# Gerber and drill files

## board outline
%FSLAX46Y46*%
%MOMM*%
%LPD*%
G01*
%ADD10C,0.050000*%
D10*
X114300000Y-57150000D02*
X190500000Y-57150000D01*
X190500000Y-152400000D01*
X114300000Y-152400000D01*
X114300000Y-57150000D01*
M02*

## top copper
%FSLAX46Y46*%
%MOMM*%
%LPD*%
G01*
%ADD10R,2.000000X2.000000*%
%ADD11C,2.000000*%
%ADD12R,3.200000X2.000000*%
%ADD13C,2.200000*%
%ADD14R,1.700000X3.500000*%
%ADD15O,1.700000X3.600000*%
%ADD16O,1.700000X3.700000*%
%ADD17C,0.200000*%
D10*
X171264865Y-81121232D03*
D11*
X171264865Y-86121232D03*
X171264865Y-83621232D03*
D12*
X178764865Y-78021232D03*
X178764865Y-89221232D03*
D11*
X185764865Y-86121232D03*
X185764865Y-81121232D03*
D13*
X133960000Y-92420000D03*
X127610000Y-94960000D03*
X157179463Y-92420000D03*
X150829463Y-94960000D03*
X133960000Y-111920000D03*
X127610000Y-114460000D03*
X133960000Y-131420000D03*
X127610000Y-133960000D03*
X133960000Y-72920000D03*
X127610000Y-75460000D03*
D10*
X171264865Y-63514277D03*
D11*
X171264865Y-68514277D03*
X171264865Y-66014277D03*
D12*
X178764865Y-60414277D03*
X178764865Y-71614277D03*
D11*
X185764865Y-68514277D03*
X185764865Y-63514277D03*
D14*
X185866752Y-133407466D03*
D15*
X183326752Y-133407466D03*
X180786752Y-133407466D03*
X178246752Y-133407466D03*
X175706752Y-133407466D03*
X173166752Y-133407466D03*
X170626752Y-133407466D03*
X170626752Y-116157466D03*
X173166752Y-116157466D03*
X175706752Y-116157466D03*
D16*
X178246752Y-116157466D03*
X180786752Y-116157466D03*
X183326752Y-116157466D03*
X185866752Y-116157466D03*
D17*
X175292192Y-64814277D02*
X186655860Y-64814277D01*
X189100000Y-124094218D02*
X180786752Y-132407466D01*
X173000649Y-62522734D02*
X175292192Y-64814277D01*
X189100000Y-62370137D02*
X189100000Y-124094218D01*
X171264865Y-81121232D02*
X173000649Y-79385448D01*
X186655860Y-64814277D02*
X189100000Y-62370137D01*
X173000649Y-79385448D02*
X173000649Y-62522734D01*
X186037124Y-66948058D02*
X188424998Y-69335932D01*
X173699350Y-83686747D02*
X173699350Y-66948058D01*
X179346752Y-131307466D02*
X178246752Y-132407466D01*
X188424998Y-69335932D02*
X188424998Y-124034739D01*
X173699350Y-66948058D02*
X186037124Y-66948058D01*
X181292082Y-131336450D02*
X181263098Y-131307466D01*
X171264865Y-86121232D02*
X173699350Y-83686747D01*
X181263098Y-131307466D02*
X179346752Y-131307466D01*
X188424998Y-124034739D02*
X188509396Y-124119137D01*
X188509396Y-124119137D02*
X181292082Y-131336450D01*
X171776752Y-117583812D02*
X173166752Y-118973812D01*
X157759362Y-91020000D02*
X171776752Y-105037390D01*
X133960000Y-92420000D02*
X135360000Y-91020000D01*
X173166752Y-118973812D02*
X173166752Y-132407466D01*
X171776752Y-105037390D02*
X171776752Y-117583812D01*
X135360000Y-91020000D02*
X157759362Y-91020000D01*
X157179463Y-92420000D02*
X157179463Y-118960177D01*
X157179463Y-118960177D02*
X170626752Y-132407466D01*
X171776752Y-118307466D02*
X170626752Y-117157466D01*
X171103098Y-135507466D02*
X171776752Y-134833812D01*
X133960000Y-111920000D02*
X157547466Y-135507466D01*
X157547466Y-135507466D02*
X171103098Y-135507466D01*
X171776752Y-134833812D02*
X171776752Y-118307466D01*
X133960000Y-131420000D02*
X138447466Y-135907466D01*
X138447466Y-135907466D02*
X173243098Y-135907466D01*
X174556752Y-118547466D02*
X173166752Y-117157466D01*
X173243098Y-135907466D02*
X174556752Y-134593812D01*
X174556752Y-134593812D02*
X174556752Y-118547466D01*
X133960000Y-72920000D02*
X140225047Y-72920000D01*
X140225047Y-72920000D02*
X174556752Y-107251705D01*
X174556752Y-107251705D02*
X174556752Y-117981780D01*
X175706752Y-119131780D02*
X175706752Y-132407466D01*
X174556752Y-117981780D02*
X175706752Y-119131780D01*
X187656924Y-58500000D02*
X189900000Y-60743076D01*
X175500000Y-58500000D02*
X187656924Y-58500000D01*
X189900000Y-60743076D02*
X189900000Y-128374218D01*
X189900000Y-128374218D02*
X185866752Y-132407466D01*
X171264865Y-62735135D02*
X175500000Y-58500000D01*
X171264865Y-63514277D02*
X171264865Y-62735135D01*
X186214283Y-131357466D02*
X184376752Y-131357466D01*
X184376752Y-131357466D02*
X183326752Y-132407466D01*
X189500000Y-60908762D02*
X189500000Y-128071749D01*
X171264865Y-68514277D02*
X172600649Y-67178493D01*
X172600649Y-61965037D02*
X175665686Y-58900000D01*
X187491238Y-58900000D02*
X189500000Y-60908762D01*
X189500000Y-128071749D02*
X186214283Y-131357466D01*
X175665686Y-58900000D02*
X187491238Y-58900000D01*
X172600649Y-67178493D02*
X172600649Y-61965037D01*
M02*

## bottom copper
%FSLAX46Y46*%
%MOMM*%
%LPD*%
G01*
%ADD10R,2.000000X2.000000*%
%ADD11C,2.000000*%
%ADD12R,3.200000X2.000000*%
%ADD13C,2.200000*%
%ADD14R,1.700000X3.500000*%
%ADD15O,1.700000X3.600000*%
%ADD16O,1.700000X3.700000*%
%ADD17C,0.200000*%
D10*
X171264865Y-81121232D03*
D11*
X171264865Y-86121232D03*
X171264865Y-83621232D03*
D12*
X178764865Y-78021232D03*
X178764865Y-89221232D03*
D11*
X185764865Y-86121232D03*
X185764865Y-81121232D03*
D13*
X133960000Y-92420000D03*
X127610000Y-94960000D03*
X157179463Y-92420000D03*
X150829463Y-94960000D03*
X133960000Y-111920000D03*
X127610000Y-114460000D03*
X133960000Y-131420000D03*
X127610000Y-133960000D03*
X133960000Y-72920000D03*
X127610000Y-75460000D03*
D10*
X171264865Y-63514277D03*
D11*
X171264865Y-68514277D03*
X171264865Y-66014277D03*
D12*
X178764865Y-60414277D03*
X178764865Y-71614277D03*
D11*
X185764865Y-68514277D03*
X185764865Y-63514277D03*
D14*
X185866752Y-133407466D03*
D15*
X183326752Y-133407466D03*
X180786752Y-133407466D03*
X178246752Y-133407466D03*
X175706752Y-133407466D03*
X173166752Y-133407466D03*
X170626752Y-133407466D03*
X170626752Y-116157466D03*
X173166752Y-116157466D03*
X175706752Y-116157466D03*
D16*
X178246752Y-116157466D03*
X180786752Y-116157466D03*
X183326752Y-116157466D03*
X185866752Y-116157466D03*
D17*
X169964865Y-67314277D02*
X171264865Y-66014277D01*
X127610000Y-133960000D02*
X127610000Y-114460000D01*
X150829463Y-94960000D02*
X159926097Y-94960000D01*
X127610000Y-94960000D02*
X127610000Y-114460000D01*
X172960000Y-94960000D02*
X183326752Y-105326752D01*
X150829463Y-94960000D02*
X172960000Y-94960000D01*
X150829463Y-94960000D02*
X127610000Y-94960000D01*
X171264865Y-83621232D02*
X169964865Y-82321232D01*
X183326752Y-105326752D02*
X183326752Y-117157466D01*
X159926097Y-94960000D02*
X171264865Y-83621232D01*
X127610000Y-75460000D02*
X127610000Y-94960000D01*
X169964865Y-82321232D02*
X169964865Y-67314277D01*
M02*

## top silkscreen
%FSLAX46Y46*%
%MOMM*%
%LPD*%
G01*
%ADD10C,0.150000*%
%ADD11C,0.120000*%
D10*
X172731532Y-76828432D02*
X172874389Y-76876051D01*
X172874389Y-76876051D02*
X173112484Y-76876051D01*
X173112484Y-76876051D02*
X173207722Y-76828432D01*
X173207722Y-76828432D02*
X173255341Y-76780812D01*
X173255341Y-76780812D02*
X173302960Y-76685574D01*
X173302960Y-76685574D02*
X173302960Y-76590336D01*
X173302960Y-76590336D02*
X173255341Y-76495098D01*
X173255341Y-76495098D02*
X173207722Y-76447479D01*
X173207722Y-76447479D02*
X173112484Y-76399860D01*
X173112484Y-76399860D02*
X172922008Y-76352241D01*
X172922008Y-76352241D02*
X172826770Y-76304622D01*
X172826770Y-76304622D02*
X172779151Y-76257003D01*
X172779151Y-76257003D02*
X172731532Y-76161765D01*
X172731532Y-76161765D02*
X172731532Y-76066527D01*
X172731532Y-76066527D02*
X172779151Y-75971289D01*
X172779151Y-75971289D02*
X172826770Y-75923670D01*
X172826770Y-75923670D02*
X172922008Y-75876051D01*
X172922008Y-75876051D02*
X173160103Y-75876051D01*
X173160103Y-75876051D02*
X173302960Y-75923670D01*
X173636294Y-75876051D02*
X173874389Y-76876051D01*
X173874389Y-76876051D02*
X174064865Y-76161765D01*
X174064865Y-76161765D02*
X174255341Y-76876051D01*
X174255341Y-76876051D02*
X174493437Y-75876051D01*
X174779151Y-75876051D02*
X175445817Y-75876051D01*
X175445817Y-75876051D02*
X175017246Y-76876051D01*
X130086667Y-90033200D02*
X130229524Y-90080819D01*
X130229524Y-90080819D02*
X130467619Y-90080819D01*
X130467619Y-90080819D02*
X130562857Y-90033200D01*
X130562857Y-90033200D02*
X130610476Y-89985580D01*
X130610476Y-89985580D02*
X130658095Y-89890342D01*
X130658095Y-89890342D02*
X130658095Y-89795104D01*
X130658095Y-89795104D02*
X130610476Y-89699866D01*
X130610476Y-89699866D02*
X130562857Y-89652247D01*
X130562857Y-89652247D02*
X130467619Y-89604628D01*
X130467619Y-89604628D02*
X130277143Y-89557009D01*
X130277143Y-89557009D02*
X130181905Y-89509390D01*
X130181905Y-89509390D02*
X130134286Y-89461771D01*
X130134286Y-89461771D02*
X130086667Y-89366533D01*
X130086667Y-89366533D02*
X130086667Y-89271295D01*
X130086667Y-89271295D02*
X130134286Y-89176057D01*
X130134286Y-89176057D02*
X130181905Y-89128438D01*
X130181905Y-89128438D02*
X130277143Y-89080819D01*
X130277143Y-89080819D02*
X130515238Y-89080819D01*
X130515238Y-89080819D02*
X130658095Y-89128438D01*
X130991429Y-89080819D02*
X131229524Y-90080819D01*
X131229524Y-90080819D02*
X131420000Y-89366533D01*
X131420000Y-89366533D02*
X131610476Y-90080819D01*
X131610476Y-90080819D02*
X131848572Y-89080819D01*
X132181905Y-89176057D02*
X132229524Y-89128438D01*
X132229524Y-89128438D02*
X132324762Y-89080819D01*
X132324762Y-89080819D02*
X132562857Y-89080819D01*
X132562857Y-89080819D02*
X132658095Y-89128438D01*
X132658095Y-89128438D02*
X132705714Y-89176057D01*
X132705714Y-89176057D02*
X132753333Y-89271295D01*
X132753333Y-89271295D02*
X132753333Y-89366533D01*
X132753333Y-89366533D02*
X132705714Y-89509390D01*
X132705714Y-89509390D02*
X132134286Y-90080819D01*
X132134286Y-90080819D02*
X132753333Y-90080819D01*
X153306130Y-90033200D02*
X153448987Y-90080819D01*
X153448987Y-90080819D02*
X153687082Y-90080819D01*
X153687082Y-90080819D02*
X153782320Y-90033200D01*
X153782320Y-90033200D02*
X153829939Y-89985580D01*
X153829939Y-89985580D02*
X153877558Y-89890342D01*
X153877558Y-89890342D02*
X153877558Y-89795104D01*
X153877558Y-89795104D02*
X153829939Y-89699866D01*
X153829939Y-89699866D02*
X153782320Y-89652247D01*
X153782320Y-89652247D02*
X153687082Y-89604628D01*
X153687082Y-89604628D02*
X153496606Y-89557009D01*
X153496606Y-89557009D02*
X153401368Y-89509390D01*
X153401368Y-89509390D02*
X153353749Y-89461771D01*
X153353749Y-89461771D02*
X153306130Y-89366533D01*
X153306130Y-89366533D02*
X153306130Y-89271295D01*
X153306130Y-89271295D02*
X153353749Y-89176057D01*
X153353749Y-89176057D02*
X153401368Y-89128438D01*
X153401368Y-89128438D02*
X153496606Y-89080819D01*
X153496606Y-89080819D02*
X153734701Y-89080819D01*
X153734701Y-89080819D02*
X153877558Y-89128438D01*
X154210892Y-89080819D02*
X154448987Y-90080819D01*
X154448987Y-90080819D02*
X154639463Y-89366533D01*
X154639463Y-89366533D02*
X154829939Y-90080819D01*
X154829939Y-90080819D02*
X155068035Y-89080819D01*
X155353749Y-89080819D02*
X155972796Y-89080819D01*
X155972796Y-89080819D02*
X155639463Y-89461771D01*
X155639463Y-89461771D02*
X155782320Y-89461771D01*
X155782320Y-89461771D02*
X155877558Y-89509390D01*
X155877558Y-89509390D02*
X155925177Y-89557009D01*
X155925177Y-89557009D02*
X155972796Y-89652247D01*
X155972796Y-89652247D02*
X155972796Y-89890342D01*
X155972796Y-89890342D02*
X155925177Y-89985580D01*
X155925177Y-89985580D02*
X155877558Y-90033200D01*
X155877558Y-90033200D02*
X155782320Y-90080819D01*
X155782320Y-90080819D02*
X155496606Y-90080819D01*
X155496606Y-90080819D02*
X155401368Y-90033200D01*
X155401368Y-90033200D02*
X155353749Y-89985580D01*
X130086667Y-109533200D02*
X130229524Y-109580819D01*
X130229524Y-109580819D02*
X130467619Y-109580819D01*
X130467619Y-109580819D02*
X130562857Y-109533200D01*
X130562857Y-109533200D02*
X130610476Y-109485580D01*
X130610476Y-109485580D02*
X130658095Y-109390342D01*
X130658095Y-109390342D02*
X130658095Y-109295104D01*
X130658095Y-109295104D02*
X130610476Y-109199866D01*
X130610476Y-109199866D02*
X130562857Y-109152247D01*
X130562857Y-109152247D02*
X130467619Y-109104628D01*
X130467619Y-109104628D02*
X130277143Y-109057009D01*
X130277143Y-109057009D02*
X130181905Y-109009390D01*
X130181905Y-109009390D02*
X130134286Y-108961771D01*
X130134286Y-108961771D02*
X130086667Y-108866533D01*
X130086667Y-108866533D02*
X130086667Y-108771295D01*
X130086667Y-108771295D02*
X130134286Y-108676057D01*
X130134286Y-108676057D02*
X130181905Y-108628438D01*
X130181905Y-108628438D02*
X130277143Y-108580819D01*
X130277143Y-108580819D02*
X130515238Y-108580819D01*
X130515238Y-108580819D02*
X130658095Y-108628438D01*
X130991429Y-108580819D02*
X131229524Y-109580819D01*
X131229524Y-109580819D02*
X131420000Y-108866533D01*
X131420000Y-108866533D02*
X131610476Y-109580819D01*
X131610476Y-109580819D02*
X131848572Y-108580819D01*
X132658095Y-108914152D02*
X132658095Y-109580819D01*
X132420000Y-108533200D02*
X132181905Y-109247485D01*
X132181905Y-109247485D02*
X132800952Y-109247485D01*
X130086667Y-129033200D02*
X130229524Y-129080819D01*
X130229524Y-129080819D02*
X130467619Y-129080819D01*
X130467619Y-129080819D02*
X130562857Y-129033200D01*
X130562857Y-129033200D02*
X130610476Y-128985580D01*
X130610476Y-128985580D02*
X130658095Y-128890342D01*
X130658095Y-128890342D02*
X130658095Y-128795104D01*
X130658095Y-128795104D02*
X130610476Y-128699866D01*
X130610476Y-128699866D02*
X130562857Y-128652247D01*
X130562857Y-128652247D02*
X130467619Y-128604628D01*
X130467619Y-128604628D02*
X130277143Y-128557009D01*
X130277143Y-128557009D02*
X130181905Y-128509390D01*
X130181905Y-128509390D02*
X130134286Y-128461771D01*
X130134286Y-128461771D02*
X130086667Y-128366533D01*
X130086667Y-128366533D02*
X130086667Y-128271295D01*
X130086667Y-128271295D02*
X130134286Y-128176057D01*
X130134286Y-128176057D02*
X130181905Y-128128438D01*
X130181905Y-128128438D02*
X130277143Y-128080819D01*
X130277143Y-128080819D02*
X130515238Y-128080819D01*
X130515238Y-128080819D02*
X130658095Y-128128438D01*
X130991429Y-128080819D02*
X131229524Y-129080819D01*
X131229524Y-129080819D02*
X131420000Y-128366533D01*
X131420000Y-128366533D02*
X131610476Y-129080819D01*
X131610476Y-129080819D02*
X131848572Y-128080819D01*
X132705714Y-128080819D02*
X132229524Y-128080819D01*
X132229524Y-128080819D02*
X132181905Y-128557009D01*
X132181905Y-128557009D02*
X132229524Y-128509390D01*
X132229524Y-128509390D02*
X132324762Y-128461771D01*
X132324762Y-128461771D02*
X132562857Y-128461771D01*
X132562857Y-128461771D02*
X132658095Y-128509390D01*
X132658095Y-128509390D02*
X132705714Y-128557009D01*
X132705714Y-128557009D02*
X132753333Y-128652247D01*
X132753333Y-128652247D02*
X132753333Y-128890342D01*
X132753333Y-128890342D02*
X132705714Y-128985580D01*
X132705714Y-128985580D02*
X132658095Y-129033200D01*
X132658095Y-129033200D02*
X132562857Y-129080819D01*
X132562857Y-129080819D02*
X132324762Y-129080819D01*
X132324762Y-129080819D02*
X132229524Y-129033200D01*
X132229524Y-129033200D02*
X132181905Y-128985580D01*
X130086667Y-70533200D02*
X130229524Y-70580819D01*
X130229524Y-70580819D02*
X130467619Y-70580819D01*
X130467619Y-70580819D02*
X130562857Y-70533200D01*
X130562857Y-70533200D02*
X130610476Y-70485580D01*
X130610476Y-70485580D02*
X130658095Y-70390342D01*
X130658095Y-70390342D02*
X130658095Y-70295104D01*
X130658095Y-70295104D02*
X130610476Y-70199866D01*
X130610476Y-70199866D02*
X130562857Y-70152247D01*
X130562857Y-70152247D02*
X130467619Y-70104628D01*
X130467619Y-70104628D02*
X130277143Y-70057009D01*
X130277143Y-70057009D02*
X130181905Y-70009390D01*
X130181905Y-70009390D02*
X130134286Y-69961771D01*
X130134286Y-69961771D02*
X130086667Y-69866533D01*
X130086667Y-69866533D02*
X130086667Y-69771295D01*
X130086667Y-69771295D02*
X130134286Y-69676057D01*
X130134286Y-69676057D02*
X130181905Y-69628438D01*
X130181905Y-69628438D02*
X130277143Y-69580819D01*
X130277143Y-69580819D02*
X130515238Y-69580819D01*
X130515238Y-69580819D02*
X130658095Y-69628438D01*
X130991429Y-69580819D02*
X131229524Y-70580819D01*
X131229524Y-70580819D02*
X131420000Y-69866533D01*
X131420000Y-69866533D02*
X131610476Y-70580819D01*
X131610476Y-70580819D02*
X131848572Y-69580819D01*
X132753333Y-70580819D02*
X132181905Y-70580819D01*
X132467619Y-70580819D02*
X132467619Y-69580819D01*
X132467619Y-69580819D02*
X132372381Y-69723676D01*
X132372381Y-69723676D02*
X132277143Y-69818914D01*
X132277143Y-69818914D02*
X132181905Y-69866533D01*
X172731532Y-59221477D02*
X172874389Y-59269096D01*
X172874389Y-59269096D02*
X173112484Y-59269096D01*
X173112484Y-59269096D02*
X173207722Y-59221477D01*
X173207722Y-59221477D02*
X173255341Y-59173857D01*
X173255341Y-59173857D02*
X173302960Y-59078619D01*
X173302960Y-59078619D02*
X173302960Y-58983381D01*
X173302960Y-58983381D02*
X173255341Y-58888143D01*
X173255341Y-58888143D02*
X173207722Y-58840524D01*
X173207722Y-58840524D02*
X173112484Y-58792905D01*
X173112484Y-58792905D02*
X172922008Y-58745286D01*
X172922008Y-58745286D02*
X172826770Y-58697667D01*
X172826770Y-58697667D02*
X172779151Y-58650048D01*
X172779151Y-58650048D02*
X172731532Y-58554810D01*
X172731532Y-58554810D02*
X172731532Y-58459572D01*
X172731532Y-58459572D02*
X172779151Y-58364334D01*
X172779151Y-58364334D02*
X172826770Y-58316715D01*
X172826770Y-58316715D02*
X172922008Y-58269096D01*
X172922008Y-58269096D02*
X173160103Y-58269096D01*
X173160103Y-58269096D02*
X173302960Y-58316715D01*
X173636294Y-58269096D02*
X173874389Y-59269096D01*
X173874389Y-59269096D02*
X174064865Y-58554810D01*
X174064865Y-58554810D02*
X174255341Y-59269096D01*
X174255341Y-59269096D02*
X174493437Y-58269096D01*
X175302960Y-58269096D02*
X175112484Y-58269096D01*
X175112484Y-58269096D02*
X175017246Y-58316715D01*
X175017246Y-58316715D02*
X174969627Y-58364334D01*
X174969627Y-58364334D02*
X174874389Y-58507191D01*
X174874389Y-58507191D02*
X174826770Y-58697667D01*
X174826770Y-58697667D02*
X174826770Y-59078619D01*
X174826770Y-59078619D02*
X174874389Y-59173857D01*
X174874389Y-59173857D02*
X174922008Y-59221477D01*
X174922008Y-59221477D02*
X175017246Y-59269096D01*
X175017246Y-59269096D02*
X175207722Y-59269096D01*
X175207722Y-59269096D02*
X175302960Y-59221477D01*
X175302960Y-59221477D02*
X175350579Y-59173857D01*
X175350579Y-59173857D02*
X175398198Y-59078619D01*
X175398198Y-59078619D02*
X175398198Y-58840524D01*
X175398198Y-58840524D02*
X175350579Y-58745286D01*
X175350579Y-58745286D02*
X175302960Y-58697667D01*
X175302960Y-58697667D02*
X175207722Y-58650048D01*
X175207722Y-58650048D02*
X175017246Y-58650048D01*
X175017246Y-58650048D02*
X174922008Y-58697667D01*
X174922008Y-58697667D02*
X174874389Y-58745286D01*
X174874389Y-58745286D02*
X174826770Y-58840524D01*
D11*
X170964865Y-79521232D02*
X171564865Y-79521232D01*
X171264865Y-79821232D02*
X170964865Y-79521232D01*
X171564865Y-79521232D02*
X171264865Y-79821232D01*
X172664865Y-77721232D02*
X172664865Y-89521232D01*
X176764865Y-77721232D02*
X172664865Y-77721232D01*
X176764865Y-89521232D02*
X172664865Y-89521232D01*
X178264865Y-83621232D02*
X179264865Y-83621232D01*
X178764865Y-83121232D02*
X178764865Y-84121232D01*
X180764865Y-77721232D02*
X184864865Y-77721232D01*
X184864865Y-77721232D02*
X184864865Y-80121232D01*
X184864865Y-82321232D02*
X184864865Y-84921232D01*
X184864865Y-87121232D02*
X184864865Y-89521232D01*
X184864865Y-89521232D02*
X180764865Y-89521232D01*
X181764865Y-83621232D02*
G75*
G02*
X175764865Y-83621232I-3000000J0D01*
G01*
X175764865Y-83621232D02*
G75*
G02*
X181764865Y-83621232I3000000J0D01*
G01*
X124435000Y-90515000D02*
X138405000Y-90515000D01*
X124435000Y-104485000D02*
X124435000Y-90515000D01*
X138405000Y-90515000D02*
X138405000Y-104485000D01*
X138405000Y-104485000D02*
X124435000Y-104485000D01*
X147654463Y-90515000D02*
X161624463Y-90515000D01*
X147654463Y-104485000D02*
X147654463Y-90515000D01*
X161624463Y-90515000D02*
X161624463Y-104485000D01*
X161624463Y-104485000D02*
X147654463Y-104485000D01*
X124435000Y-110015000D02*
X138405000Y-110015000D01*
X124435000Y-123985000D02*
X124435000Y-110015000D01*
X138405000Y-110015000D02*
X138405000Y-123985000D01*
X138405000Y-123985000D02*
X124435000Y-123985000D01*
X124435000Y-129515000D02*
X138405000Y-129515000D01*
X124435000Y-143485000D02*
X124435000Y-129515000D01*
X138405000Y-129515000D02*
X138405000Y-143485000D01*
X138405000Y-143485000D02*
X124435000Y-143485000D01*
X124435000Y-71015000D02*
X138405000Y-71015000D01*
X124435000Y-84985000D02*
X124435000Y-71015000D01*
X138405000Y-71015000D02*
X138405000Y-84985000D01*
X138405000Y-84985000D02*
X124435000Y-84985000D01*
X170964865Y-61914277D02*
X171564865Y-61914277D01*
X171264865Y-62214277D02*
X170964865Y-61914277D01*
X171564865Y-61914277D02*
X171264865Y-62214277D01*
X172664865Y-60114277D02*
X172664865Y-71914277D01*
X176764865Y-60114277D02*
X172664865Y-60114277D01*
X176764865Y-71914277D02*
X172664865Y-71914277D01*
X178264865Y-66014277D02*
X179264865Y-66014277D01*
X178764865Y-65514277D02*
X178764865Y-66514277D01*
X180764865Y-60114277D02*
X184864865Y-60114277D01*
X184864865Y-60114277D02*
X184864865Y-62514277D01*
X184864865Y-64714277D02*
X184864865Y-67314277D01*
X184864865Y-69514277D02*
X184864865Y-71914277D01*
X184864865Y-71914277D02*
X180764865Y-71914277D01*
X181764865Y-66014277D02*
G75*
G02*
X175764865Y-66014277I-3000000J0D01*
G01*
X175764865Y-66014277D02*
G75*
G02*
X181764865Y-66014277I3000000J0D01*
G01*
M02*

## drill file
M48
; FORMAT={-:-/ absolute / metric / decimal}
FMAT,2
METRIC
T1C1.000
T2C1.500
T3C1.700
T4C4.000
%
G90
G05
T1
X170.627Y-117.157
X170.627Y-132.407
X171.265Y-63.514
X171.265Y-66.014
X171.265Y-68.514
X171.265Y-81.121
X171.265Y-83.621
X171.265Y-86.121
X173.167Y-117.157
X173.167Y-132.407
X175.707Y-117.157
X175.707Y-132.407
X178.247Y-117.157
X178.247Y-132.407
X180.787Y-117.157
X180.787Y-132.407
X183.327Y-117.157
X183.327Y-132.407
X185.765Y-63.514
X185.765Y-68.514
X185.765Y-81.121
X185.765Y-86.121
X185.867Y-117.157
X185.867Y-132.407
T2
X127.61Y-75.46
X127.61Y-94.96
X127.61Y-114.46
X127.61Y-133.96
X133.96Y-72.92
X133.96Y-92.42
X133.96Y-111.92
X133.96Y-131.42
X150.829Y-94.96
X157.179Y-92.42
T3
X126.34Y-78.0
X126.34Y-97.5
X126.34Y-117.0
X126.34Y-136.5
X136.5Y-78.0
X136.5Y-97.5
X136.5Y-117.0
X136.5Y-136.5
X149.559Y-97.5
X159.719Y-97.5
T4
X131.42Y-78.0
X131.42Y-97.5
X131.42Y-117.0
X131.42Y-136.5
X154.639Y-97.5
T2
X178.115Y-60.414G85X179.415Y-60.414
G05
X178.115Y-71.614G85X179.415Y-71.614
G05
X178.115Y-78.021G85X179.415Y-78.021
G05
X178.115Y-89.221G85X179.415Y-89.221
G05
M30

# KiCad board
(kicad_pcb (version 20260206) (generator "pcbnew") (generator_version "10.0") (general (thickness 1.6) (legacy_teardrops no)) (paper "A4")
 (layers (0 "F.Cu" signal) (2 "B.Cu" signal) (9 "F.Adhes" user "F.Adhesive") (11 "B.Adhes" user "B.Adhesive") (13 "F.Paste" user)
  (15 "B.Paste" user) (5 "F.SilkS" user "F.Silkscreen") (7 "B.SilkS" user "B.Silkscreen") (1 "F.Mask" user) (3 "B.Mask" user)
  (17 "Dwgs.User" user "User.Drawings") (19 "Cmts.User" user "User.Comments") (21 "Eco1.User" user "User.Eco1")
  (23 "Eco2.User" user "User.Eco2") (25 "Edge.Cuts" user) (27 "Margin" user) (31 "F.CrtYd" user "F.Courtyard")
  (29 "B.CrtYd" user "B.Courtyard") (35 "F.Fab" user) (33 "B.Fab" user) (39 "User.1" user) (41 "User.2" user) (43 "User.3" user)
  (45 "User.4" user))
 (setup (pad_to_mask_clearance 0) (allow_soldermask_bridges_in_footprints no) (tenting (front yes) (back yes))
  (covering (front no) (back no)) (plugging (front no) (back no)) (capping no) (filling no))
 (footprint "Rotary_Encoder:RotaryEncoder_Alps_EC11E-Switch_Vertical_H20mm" (layer "F.Cu") (at 171.264865 81.121232)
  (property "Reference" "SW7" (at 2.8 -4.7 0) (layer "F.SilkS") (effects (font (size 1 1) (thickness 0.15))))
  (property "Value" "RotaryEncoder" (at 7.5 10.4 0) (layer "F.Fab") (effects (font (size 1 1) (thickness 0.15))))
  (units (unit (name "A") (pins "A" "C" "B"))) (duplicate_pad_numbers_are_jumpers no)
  (fp_line (start -0.3 -1.6) (end 0.3 -1.6) (stroke (width 0.12) (type solid)) (layer "F.SilkS"))
  (fp_line (start 0 -1.3) (end -0.3 -1.6) (stroke (width 0.12) (type solid)) (layer "F.SilkS"))
  (fp_line (start 0.3 -1.6) (end 0 -1.3) (stroke (width 0.12) (type solid)) (layer "F.SilkS"))
  (fp_line (start 1.4 -3.4) (end 1.4 8.4) (stroke (width 0.12) (type solid)) (layer "F.SilkS"))
  (fp_line (start 5.5 -3.4) (end 1.4 -3.4) (stroke (width 0.12) (type solid)) (layer "F.SilkS"))
  (fp_line (start 5.5 8.4) (end 1.4 8.4) (stroke (width 0.12) (type solid)) (layer "F.SilkS"))
  (fp_line (start 7 2.5) (end 8 2.5) (stroke (width 0.12) (type solid)) (layer "F.SilkS"))
  (fp_line (start 7.5 2) (end 7.5 3) (stroke (width 0.12) (type solid)) (layer "F.SilkS"))
  (fp_line (start 9.5 -3.4) (end 13.6 -3.4) (stroke (width 0.12) (type solid)) (layer "F.SilkS"))
  (fp_line (start 13.6 -3.4) (end 13.6 -1) (stroke (width 0.12) (type solid)) (layer "F.SilkS"))
  (fp_line (start 13.6 1.2) (end 13.6 3.8) (stroke (width 0.12) (type solid)) (layer "F.SilkS"))
  (fp_line (start 13.6 6) (end 13.6 8.4) (stroke (width 0.12) (type solid)) (layer "F.SilkS"))
  (fp_line (start 13.6 8.4) (end 9.5 8.4) (stroke (width 0.12) (type solid)) (layer "F.SilkS"))
  (fp_circle (center 7.5 2.5) (end 10.5 2.5) (stroke (width 0.12) (type solid)) (fill no) (layer "F.SilkS"))
  (pad "A" thru_hole rect (at 0 0) (size 2 2) (drill 1) (layers "*.Cu" "*.Mask") (remove_unused_layers no) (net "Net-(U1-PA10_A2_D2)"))
  (pad "B" thru_hole circle (at 0 5) (size 2 2) (drill 1) (layers "*.Cu" "*.Mask") (remove_unused_layers no) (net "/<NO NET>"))
  (pad "C" thru_hole circle (at 0 2.5) (size 2 2) (drill 1) (layers "*.Cu" "*.Mask") (remove_unused_layers no) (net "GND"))
  (pad "MP" thru_hole rect (at 7.5 -3.1) (size 3.2 2) (drill oval 2.8 1.5) (layers "*.Cu" "*.Mask") (remove_unused_layers no))
  (pad "MP" thru_hole rect (at 7.5 8.1) (size 3.2 2) (drill oval 2.8 1.5) (layers "*.Cu" "*.Mask") (remove_unused_layers no))
  (pad "S1" thru_hole circle (at 14.5 5) (size 2 2) (drill 1) (layers "*.Cu" "*.Mask") (remove_unused_layers no))
  (pad "S2" thru_hole circle (at 14.5 0) (size 2 2) (drill 1) (layers "*.Cu" "*.Mask") (remove_unused_layers no)))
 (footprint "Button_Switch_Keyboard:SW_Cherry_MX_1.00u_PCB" (layer "F.Cu") (at 133.96 92.42)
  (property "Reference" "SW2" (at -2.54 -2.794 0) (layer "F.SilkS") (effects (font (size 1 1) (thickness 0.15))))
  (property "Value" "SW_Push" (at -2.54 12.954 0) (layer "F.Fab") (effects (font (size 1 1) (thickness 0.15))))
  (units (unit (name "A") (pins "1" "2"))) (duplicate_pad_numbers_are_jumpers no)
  (fp_line (start -9.525 -1.905) (end 4.445 -1.905) (stroke (width 0.12) (type solid)) (layer "F.SilkS"))
  (fp_line (start -9.525 12.065) (end -9.525 -1.905) (stroke (width 0.12) (type solid)) (layer "F.SilkS"))
  (fp_line (start 4.445 -1.905) (end 4.445 12.065) (stroke (width 0.12) (type solid)) (layer "F.SilkS"))
  (fp_line (start 4.445 12.065) (end -9.525 12.065) (stroke (width 0.12) (type solid)) (layer "F.SilkS"))
  (pad "" np_thru_hole circle (at -7.62 5.08) (size 1.7 1.7) (drill 1.7) (layers "*.Cu" "*.Mask"))
  (pad "" np_thru_hole circle (at -2.54 5.08) (size 4 4) (drill 4) (layers "*.Cu" "*.Mask"))
  (pad "" np_thru_hole circle (at 2.54 5.08) (size 1.7 1.7) (drill 1.7) (layers "*.Cu" "*.Mask"))
  (pad "1" thru_hole circle (at 0 0) (size 2.2 2.2) (drill 1.5) (layers "*.Cu" "*.Mask") (remove_unused_layers no)
   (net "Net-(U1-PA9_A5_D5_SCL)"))
  (pad "2" thru_hole circle (at -6.35 2.54) (size 2.2 2.2) (drill 1.5) (layers "*.Cu" "*.Mask") (remove_unused_layers no) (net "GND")))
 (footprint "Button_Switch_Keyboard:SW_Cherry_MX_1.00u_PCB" (layer "F.Cu") (at 157.179463 92.42)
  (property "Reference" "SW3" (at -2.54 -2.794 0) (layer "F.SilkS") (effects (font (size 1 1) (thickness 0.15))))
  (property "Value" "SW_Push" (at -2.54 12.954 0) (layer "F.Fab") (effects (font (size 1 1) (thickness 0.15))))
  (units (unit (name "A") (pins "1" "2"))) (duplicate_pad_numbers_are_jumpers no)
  (fp_line (start -9.525 -1.905) (end 4.445 -1.905) (stroke (width 0.12) (type solid)) (layer "F.SilkS"))
  (fp_line (start -9.525 12.065) (end -9.525 -1.905) (stroke (width 0.12) (type solid)) (layer "F.SilkS"))
  (fp_line (start 4.445 -1.905) (end 4.445 12.065) (stroke (width 0.12) (type solid)) (layer "F.SilkS"))
  (fp_line (start 4.445 12.065) (end -9.525 12.065) (stroke (width 0.12) (type solid)) (layer "F.SilkS"))
  (pad "" np_thru_hole circle (at -7.62 5.08) (size 1.7 1.7) (drill 1.7) (layers "*.Cu" "*.Mask"))
  (pad "" np_thru_hole circle (at -2.54 5.08) (size 4 4) (drill 4) (layers "*.Cu" "*.Mask"))
  (pad "" np_thru_hole circle (at 2.54 5.08) (size 1.7 1.7) (drill 1.7) (layers "*.Cu" "*.Mask"))
  (pad "1" thru_hole circle (at 0 0) (size 2.2 2.2) (drill 1.5) (layers "*.Cu" "*.Mask") (remove_unused_layers no)
   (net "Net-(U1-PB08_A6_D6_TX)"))
  (pad "2" thru_hole circle (at -6.35 2.54) (size 2.2 2.2) (drill 1.5) (layers "*.Cu" "*.Mask") (remove_unused_layers no) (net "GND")))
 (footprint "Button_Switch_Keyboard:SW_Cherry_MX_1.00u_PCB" (layer "F.Cu") (at 133.96 111.92)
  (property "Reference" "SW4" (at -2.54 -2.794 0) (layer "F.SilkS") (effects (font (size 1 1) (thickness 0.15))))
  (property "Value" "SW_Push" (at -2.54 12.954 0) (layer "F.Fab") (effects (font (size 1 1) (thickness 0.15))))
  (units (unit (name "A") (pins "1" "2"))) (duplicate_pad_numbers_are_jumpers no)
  (fp_line (start -9.525 -1.905) (end 4.445 -1.905) (stroke (width 0.12) (type solid)) (layer "F.SilkS"))
  (fp_line (start -9.525 12.065) (end -9.525 -1.905) (stroke (width 0.12) (type solid)) (layer "F.SilkS"))
  (fp_line (start 4.445 -1.905) (end 4.445 12.065) (stroke (width 0.12) (type solid)) (layer "F.SilkS"))
  (fp_line (start 4.445 12.065) (end -9.525 12.065) (stroke (width 0.12) (type solid)) (layer "F.SilkS"))
  (pad "" np_thru_hole circle (at -7.62 5.08) (size 1.7 1.7) (drill 1.7) (layers "*.Cu" "*.Mask"))
  (pad "" np_thru_hole circle (at -2.54 5.08) (size 4 4) (drill 4) (layers "*.Cu" "*.Mask"))
  (pad "" np_thru_hole circle (at 2.54 5.08) (size 1.7 1.7) (drill 1.7) (layers "*.Cu" "*.Mask"))
  (pad "1" thru_hole circle (at 0 0) (size 2.2 2.2) (drill 1.5) (layers "*.Cu" "*.Mask") (remove_unused_layers no)
   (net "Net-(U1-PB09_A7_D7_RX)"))
  (pad "2" thru_hole circle (at -6.35 2.54) (size 2.2 2.2) (drill 1.5) (layers "*.Cu" "*.Mask") (remove_unused_layers no) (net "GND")))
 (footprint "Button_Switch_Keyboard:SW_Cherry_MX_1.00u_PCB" (layer "F.Cu") (at 133.96 131.42)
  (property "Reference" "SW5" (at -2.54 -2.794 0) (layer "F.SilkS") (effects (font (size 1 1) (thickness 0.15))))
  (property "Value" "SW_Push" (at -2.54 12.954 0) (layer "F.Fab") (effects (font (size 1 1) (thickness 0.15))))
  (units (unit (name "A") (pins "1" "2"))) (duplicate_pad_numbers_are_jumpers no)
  (fp_line (start -9.525 -1.905) (end 4.445 -1.905) (stroke (width 0.12) (type solid)) (layer "F.SilkS"))
  (fp_line (start -9.525 12.065) (end -9.525 -1.905) (stroke (width 0.12) (type solid)) (layer "F.SilkS"))
  (fp_line (start 4.445 -1.905) (end 4.445 12.065) (stroke (width 0.12) (type solid)) (layer "F.SilkS"))
  (fp_line (start 4.445 12.065) (end -9.525 12.065) (stroke (width 0.12) (type solid)) (layer "F.SilkS"))
  (pad "" np_thru_hole circle (at -7.62 5.08) (size 1.7 1.7) (drill 1.7) (layers "*.Cu" "*.Mask"))
  (pad "" np_thru_hole circle (at -2.54 5.08) (size 4 4) (drill 4) (layers "*.Cu" "*.Mask"))
  (pad "" np_thru_hole circle (at 2.54 5.08) (size 1.7 1.7) (drill 1.7) (layers "*.Cu" "*.Mask"))
  (pad "1" thru_hole circle (at 0 0) (size 2.2 2.2) (drill 1.5) (layers "*.Cu" "*.Mask") (remove_unused_layers no)
   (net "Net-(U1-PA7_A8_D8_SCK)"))
  (pad "2" thru_hole circle (at -6.35 2.54) (size 2.2 2.2) (drill 1.5) (layers "*.Cu" "*.Mask") (remove_unused_layers no) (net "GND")))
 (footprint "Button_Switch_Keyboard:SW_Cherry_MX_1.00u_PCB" (layer "F.Cu") (at 133.96 72.92)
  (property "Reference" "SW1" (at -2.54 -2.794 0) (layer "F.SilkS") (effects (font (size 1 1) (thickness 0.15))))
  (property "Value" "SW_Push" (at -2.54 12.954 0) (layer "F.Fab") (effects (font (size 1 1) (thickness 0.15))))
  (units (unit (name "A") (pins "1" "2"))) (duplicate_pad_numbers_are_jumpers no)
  (fp_line (start -9.525 -1.905) (end 4.445 -1.905) (stroke (width 0.12) (type solid)) (layer "F.SilkS"))
  (fp_line (start -9.525 12.065) (end -9.525 -1.905) (stroke (width 0.12) (type solid)) (layer "F.SilkS"))
  (fp_line (start 4.445 -1.905) (end 4.445 12.065) (stroke (width 0.12) (type solid)) (layer "F.SilkS"))
  (fp_line (start 4.445 12.065) (end -9.525 12.065) (stroke (width 0.12) (type solid)) (layer "F.SilkS"))
  (pad "" np_thru_hole circle (at -7.62 5.08) (size 1.7 1.7) (drill 1.7) (layers "*.Cu" "*.Mask"))
  (pad "" np_thru_hole circle (at -2.54 5.08) (size 4 4) (drill 4) (layers "*.Cu" "*.Mask"))
  (pad "" np_thru_hole circle (at 2.54 5.08) (size 1.7 1.7) (drill 1.7) (layers "*.Cu" "*.Mask"))
  (pad "1" thru_hole circle (at 0 0) (size 2.2 2.2) (drill 1.5) (layers "*.Cu" "*.Mask") (remove_unused_layers no)
   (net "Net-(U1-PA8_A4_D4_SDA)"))
  (pad "2" thru_hole circle (at -6.35 2.54) (size 2.2 2.2) (drill 1.5) (layers "*.Cu" "*.Mask") (remove_unused_layers no) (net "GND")))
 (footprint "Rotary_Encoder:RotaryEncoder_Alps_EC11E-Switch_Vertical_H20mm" (layer "F.Cu") (at 171.264865 63.514277)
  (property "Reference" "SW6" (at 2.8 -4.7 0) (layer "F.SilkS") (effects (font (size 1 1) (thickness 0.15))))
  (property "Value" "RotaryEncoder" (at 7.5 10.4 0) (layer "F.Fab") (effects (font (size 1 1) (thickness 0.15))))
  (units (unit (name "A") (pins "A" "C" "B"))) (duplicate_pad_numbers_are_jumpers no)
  (fp_line (start -0.3 -1.6) (end 0.3 -1.6) (stroke (width 0.12) (type solid)) (layer "F.SilkS"))
  (fp_line (start 0 -1.3) (end -0.3 -1.6) (stroke (width 0.12) (type solid)) (layer "F.SilkS"))
  (fp_line (start 0.3 -1.6) (end 0 -1.3) (stroke (width 0.12) (type solid)) (layer "F.SilkS"))
  (fp_line (start 1.4 -3.4) (end 1.4 8.4) (stroke (width 0.12) (type solid)) (layer "F.SilkS"))
  (fp_line (start 5.5 -3.4) (end 1.4 -3.4) (stroke (width 0.12) (type solid)) (layer "F.SilkS"))
  (fp_line (start 5.5 8.4) (end 1.4 8.4) (stroke (width 0.12) (type solid)) (layer "F.SilkS"))
  (fp_line (start 7 2.5) (end 8 2.5) (stroke (width 0.12) (type solid)) (layer "F.SilkS"))
  (fp_line (start 7.5 2) (end 7.5 3) (stroke (width 0.12) (type solid)) (layer "F.SilkS"))
  (fp_line (start 9.5 -3.4) (end 13.6 -3.4) (stroke (width 0.12) (type solid)) (layer "F.SilkS"))
  (fp_line (start 13.6 -3.4) (end 13.6 -1) (stroke (width 0.12) (type solid)) (layer "F.SilkS"))
  (fp_line (start 13.6 1.2) (end 13.6 3.8) (stroke (width 0.12) (type solid)) (layer "F.SilkS"))
  (fp_line (start 13.6 6) (end 13.6 8.4) (stroke (width 0.12) (type solid)) (layer "F.SilkS"))
  (fp_line (start 13.6 8.4) (end 9.5 8.4) (stroke (width 0.12) (type solid)) (layer "F.SilkS"))
  (fp_circle (center 7.5 2.5) (end 10.5 2.5) (stroke (width 0.12) (type solid)) (fill no) (layer "F.SilkS"))
  (pad "A" thru_hole rect (at 0 0) (size 2 2) (drill 1) (layers "*.Cu" "*.Mask") (remove_unused_layers no) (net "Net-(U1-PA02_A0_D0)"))
  (pad "B" thru_hole circle (at 0 5) (size 2 2) (drill 1) (layers "*.Cu" "*.Mask") (remove_unused_layers no) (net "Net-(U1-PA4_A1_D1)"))
  (pad "C" thru_hole circle (at 0 2.5) (size 2 2) (drill 1) (layers "*.Cu" "*.Mask") (remove_unused_layers no) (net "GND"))
  (pad "MP" thru_hole rect (at 7.5 -3.1) (size 3.2 2) (drill oval 2.8 1.5) (layers "*.Cu" "*.Mask") (remove_unused_layers no))
  (pad "MP" thru_hole rect (at 7.5 8.1) (size 3.2 2) (drill oval 2.8 1.5) (layers "*.Cu" "*.Mask") (remove_unused_layers no))
  (pad "S1" thru_hole circle (at 14.5 5) (size 2 2) (drill 1) (layers "*.Cu" "*.Mask") (remove_unused_layers no))
  (pad "S2" thru_hole circle (at 14.5 0) (size 2 2) (drill 1) (layers "*.Cu" "*.Mask") (remove_unused_layers no)))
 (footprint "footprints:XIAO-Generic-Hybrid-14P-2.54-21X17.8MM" (layer "B.Cu") (at 178.246752 124.782466 90)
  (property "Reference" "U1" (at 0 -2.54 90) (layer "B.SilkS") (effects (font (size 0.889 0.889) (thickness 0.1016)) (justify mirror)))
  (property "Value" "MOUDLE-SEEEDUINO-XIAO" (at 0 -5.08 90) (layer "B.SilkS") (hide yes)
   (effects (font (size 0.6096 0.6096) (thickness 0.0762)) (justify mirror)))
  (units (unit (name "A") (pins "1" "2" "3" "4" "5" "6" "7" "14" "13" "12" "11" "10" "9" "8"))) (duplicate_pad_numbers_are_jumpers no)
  (pad "1" thru_hole rect (at -7.625 7.62 90) (size 3.5 1.7) (drill 1 (offset -1 0)) (layers "*.Cu" "*.Mask") (remove_unused_layers no)
   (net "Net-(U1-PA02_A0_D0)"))
  (pad "2" thru_hole oval (at -7.625 5.08 90) (size 3.6 1.7) (drill 1 (offset -1 0)) (layers "*.Cu" "*.Mask") (remove_unused_layers no)
   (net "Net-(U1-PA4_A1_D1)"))
  (pad "3" thru_hole oval (at -7.625 2.54 90) (size 3.6 1.7) (drill 1 (offset -1 0)) (layers "*.Cu" "*.Mask") (remove_unused_layers no)
   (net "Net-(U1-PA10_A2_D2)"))
  (pad "4" thru_hole oval (at -7.625 0 90) (size 3.6 1.7) (drill 1 (offset -1 0)) (layers "*.Cu" "*.Mask") (remove_unused_layers no)
   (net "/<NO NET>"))
  (pad "5" thru_hole oval (at -7.625 -2.54 90) (size 3.6 1.7) (drill 1 (offset -1 0)) (layers "*.Cu" "*.Mask") (remove_unused_layers no)
   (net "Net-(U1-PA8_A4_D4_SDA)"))
  (pad "6" thru_hole oval (at -7.625 -5.08 270) (size 3.6 1.7) (drill 1 (offset 1 0)) (layers "*.Cu" "*.Mask") (remove_unused_layers no)
   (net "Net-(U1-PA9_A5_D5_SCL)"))
  (pad "7" thru_hole oval (at -7.625 -7.62 90) (size 3.6 1.7) (drill 1 (offset -1 0)) (layers "*.Cu" "*.Mask") (remove_unused_layers no)
   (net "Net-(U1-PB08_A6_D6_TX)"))
  (pad "8" thru_hole oval (at 7.625 -7.62 90) (size 3.6 1.7) (drill 1 (offset 1 0)) (layers "*.Cu" "*.Mask") (remove_unused_layers no)
   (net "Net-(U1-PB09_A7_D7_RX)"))
  (pad "9" thru_hole oval (at 7.625 -5.08 90) (size 3.6 1.7) (drill 1 (offset 1 0)) (layers "*.Cu" "*.Mask") (remove_unused_layers no)
   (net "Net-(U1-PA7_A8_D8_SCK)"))
  (pad "10" thru_hole oval (at 7.625 -2.54 90) (size 3.6 1.7) (drill 1 (offset 1 0)) (layers "*.Cu" "*.Mask") (remove_unused_layers no)
   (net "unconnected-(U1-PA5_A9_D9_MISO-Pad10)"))
  (pad "11" thru_hole oval (at 7.625 0 90) (size 3.7 1.7) (drill 1 (offset 1 0)) (layers "*.Cu" "*.Mask") (remove_unused_layers no)
   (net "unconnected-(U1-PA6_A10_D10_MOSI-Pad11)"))
  (pad "12" thru_hole oval (at 7.625 2.54 90) (size 3.7 1.7) (drill 1 (offset 1 0)) (layers "*.Cu" "*.Mask") (remove_unused_layers no)
   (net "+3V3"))
  (pad "13" thru_hole oval (at 7.625 5.08 90) (size 3.7 1.7) (drill 1 (offset 1 0)) (layers "*.Cu" "*.Mask") (remove_unused_layers no)
   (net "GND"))
  (pad "14" thru_hole oval (at 7.625 7.62 90) (size 3.7 1.7) (drill 1 (offset 1 0)) (layers "*.Cu" "*.Mask") (remove_unused_layers no)
   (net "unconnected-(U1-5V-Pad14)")))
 (gr_rect (start 114.3 57.15) (end 190.5 152.4) (stroke (width 0.05) (type default)) (fill no) (layer "Edge.Cuts"))
 (segment (start 175.292192 64.814277) (end 186.65586 64.814277) (width 0.2) (layer "F.Cu") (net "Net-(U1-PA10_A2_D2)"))
 (segment (start 189.1 124.094218) (end 180.786752 132.407466) (width 0.2) (layer "F.Cu") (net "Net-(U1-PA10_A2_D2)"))
 (segment (start 173.000649 62.522734) (end 175.292192 64.814277) (width 0.2) (layer "F.Cu") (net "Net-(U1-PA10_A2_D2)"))
 (segment (start 189.1 62.370137) (end 189.1 124.094218) (width 0.2) (layer "F.Cu") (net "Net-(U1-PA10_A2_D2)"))
 (segment (start 171.264865 81.121232) (end 173.000649 79.385448) (width 0.2) (layer "F.Cu") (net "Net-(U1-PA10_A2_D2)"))
 (segment (start 186.65586 64.814277) (end 189.1 62.370137) (width 0.2) (layer "F.Cu") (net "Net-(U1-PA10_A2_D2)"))
 (segment (start 173.000649 79.385448) (end 173.000649 62.522734) (width 0.2) (layer "F.Cu") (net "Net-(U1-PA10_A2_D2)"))
 (segment (start 186.037124 66.948058) (end 188.424998 69.335932) (width 0.2) (layer "F.Cu") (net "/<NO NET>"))
 (segment (start 173.69935 83.686747) (end 173.69935 66.948058) (width 0.2) (layer "F.Cu") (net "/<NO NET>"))
 (segment (start 179.346752 131.307466) (end 178.246752 132.407466) (width 0.2) (layer "F.Cu") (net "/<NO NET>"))
 (segment (start 188.424998 69.335932) (end 188.424998 124.034739) (width 0.2) (layer "F.Cu") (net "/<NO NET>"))
 (segment (start 173.69935 66.948058) (end 186.037124 66.948058) (width 0.2) (layer "F.Cu") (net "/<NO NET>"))
 (segment (start 181.292082 131.33645) (end 181.263098 131.307466) (width 0.2) (layer "F.Cu") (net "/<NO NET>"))
 (segment (start 171.264865 86.121232) (end 173.69935 83.686747) (width 0.2) (layer "F.Cu") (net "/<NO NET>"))
 (segment (start 181.263098 131.307466) (end 179.346752 131.307466) (width 0.2) (layer "F.Cu") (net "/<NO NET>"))
 (segment (start 188.424998 124.034739) (end 188.509396 124.119137) (width 0.2) (layer "F.Cu") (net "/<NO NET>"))
 (segment (start 188.509396 124.119137) (end 181.292082 131.33645) (width 0.2) (layer "F.Cu") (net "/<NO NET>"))
 (segment (start 169.964865 67.314277) (end 171.264865 66.014277) (width 0.2) (layer "B.Cu") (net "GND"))
 (segment (start 127.61 133.96) (end 127.61 114.46) (width 0.2) (layer "B.Cu") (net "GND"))
 (segment (start 150.829463 94.96) (end 159.926097 94.96) (width 0.2) (layer "B.Cu") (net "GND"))
 (segment (start 127.61 94.96) (end 127.61 114.46) (width 0.2) (layer "B.Cu") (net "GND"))
 (segment (start 172.96 94.96) (end 183.326752 105.326752) (width 0.2) (layer "B.Cu") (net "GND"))
 (segment (start 150.829463 94.96) (end 172.96 94.96) (width 0.2) (layer "B.Cu") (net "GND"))
 (segment (start 150.829463 94.96) (end 127.61 94.96) (width 0.2) (layer "B.Cu") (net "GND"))
 (segment (start 171.264865 83.621232) (end 169.964865 82.321232) (width 0.2) (layer "B.Cu") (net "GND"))
 (segment (start 183.326752 105.326752) (end 183.326752 117.157466) (width 0.2) (layer "B.Cu") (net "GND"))
 (segment (start 159.926097 94.96) (end 171.264865 83.621232) (width 0.2) (layer "B.Cu") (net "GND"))
 (segment (start 127.61 75.46) (end 127.61 94.96) (width 0.2) (layer "B.Cu") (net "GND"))
 (segment (start 169.964865 82.321232) (end 169.964865 67.314277) (width 0.2) (layer "B.Cu") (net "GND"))
 (segment (start 171.776752 117.583812) (end 173.166752 118.973812) (width 0.2) (layer "F.Cu") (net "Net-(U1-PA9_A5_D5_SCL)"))
 (segment (start 157.759362 91.02) (end 171.776752 105.03739) (width 0.2) (layer "F.Cu") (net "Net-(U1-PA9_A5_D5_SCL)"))
 (segment (start 133.96 92.42) (end 135.36 91.02) (width 0.2) (layer "F.Cu") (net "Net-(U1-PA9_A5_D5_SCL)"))
 (segment (start 173.166752 118.973812) (end 173.166752 132.407466) (width 0.2) (layer "F.Cu") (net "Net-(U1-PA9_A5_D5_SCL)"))
 (segment (start 171.776752 105.03739) (end 171.776752 117.583812) (width 0.2) (layer "F.Cu") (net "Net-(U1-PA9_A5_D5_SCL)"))
 (segment (start 135.36 91.02) (end 157.759362 91.02) (width 0.2) (layer "F.Cu") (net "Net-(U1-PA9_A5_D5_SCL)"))
 (segment (start 157.179463 92.42) (end 157.179463 118.960177) (width 0.2) (layer "F.Cu") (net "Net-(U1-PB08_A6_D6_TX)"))
 (segment (start 157.179463 118.960177) (end 170.626752 132.407466) (width 0.2) (layer "F.Cu") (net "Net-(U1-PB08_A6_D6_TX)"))
 (segment (start 171.776752 118.307466) (end 170.626752 117.157466) (width 0.2) (layer "F.Cu") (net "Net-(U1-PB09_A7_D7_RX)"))
 (segment (start 171.103098 135.507466) (end 171.776752 134.833812) (width 0.2) (layer "F.Cu") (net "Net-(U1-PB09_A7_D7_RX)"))
 (segment (start 133.96 111.92) (end 157.547466 135.507466) (width 0.2) (layer "F.Cu") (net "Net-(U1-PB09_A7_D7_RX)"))
 (segment (start 157.547466 135.507466) (end 171.103098 135.507466) (width 0.2) (layer "F.Cu") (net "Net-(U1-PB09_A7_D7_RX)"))
 (segment (start 171.776752 134.833812) (end 171.776752 118.307466) (width 0.2) (layer "F.Cu") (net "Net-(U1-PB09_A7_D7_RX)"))
 (segment (start 133.96 131.42) (end 138.447466 135.907466) (width 0.2) (layer "F.Cu") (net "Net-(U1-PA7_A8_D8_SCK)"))
 (segment (start 138.447466 135.907466) (end 173.243098 135.907466) (width 0.2) (layer "F.Cu") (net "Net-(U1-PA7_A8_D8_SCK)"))
 (segment (start 174.556752 118.547466) (end 173.166752 117.157466) (width 0.2) (layer "F.Cu") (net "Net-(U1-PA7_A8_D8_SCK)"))
 (segment (start 173.243098 135.907466) (end 174.556752 134.593812) (width 0.2) (layer "F.Cu") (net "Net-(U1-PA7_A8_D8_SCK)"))
 (segment (start 174.556752 134.593812) (end 174.556752 118.547466) (width 0.2) (layer "F.Cu") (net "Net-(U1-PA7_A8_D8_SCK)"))
 (segment (start 133.96 72.92) (end 140.225047 72.92) (width 0.2) (layer "F.Cu") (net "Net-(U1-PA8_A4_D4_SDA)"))
 (segment (start 140.225047 72.92) (end 174.556752 107.251705) (width 0.2) (layer "F.Cu") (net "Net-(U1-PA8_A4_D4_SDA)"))
 (segment (start 174.556752 107.251705) (end 174.556752 117.98178) (width 0.2) (layer "F.Cu") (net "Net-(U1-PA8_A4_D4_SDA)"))
 (segment (start 175.706752 119.13178) (end 175.706752 132.407466) (width 0.2) (layer "F.Cu") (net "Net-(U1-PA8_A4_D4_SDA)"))
 (segment (start 174.556752 117.98178) (end 175.706752 119.13178) (width 0.2) (layer "F.Cu") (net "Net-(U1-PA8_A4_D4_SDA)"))
 (segment (start 187.656924 58.5) (end 189.9 60.743076) (width 0.2) (layer "F.Cu") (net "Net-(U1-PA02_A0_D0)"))
 (segment (start 175.5 58.5) (end 187.656924 58.5) (width 0.2) (layer "F.Cu") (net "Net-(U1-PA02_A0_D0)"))
 (segment (start 189.9 60.743076) (end 189.9 128.374218) (width 0.2) (layer "F.Cu") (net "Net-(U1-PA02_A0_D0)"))
 (segment (start 189.9 128.374218) (end 185.866752 132.407466) (width 0.2) (layer "F.Cu") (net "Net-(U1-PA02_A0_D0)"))
 (segment (start 171.264865 62.735135) (end 175.5 58.5) (width 0.2) (layer "F.Cu") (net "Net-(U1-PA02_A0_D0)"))
 (segment (start 171.264865 63.514277) (end 171.264865 62.735135) (width 0.2) (layer "F.Cu") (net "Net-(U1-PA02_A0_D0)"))
 (segment (start 186.214283 131.357466) (end 184.376752 131.357466) (width 0.2) (layer "F.Cu") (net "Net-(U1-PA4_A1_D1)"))
 (segment (start 184.376752 131.357466) (end 183.326752 132.407466) (width 0.2) (layer "F.Cu") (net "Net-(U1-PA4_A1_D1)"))
 (segment (start 189.5 60.908762) (end 189.5 128.071749) (width 0.2) (layer "F.Cu") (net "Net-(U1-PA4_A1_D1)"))
 (segment (start 171.264865 68.514277) (end 172.600649 67.178493) (width 0.2) (layer "F.Cu") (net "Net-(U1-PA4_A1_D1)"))
 (segment (start 172.600649 61.965037) (end 175.665686 58.9) (width 0.2) (layer "F.Cu") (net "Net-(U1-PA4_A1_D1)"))
 (segment (start 187.491238 58.9) (end 189.5 60.908762) (width 0.2) (layer "F.Cu") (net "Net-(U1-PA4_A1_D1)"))
 (segment (start 189.5 128.071749) (end 186.214283 131.357466) (width 0.2) (layer "F.Cu") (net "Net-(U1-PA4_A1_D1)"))
 (segment (start 175.665686 58.9) (end 187.491238 58.9) (width 0.2) (layer "F.Cu") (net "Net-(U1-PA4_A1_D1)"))
 (segment (start 172.600649 67.178493) (end 172.600649 61.965037) (width 0.2) (layer "F.Cu") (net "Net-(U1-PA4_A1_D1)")))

